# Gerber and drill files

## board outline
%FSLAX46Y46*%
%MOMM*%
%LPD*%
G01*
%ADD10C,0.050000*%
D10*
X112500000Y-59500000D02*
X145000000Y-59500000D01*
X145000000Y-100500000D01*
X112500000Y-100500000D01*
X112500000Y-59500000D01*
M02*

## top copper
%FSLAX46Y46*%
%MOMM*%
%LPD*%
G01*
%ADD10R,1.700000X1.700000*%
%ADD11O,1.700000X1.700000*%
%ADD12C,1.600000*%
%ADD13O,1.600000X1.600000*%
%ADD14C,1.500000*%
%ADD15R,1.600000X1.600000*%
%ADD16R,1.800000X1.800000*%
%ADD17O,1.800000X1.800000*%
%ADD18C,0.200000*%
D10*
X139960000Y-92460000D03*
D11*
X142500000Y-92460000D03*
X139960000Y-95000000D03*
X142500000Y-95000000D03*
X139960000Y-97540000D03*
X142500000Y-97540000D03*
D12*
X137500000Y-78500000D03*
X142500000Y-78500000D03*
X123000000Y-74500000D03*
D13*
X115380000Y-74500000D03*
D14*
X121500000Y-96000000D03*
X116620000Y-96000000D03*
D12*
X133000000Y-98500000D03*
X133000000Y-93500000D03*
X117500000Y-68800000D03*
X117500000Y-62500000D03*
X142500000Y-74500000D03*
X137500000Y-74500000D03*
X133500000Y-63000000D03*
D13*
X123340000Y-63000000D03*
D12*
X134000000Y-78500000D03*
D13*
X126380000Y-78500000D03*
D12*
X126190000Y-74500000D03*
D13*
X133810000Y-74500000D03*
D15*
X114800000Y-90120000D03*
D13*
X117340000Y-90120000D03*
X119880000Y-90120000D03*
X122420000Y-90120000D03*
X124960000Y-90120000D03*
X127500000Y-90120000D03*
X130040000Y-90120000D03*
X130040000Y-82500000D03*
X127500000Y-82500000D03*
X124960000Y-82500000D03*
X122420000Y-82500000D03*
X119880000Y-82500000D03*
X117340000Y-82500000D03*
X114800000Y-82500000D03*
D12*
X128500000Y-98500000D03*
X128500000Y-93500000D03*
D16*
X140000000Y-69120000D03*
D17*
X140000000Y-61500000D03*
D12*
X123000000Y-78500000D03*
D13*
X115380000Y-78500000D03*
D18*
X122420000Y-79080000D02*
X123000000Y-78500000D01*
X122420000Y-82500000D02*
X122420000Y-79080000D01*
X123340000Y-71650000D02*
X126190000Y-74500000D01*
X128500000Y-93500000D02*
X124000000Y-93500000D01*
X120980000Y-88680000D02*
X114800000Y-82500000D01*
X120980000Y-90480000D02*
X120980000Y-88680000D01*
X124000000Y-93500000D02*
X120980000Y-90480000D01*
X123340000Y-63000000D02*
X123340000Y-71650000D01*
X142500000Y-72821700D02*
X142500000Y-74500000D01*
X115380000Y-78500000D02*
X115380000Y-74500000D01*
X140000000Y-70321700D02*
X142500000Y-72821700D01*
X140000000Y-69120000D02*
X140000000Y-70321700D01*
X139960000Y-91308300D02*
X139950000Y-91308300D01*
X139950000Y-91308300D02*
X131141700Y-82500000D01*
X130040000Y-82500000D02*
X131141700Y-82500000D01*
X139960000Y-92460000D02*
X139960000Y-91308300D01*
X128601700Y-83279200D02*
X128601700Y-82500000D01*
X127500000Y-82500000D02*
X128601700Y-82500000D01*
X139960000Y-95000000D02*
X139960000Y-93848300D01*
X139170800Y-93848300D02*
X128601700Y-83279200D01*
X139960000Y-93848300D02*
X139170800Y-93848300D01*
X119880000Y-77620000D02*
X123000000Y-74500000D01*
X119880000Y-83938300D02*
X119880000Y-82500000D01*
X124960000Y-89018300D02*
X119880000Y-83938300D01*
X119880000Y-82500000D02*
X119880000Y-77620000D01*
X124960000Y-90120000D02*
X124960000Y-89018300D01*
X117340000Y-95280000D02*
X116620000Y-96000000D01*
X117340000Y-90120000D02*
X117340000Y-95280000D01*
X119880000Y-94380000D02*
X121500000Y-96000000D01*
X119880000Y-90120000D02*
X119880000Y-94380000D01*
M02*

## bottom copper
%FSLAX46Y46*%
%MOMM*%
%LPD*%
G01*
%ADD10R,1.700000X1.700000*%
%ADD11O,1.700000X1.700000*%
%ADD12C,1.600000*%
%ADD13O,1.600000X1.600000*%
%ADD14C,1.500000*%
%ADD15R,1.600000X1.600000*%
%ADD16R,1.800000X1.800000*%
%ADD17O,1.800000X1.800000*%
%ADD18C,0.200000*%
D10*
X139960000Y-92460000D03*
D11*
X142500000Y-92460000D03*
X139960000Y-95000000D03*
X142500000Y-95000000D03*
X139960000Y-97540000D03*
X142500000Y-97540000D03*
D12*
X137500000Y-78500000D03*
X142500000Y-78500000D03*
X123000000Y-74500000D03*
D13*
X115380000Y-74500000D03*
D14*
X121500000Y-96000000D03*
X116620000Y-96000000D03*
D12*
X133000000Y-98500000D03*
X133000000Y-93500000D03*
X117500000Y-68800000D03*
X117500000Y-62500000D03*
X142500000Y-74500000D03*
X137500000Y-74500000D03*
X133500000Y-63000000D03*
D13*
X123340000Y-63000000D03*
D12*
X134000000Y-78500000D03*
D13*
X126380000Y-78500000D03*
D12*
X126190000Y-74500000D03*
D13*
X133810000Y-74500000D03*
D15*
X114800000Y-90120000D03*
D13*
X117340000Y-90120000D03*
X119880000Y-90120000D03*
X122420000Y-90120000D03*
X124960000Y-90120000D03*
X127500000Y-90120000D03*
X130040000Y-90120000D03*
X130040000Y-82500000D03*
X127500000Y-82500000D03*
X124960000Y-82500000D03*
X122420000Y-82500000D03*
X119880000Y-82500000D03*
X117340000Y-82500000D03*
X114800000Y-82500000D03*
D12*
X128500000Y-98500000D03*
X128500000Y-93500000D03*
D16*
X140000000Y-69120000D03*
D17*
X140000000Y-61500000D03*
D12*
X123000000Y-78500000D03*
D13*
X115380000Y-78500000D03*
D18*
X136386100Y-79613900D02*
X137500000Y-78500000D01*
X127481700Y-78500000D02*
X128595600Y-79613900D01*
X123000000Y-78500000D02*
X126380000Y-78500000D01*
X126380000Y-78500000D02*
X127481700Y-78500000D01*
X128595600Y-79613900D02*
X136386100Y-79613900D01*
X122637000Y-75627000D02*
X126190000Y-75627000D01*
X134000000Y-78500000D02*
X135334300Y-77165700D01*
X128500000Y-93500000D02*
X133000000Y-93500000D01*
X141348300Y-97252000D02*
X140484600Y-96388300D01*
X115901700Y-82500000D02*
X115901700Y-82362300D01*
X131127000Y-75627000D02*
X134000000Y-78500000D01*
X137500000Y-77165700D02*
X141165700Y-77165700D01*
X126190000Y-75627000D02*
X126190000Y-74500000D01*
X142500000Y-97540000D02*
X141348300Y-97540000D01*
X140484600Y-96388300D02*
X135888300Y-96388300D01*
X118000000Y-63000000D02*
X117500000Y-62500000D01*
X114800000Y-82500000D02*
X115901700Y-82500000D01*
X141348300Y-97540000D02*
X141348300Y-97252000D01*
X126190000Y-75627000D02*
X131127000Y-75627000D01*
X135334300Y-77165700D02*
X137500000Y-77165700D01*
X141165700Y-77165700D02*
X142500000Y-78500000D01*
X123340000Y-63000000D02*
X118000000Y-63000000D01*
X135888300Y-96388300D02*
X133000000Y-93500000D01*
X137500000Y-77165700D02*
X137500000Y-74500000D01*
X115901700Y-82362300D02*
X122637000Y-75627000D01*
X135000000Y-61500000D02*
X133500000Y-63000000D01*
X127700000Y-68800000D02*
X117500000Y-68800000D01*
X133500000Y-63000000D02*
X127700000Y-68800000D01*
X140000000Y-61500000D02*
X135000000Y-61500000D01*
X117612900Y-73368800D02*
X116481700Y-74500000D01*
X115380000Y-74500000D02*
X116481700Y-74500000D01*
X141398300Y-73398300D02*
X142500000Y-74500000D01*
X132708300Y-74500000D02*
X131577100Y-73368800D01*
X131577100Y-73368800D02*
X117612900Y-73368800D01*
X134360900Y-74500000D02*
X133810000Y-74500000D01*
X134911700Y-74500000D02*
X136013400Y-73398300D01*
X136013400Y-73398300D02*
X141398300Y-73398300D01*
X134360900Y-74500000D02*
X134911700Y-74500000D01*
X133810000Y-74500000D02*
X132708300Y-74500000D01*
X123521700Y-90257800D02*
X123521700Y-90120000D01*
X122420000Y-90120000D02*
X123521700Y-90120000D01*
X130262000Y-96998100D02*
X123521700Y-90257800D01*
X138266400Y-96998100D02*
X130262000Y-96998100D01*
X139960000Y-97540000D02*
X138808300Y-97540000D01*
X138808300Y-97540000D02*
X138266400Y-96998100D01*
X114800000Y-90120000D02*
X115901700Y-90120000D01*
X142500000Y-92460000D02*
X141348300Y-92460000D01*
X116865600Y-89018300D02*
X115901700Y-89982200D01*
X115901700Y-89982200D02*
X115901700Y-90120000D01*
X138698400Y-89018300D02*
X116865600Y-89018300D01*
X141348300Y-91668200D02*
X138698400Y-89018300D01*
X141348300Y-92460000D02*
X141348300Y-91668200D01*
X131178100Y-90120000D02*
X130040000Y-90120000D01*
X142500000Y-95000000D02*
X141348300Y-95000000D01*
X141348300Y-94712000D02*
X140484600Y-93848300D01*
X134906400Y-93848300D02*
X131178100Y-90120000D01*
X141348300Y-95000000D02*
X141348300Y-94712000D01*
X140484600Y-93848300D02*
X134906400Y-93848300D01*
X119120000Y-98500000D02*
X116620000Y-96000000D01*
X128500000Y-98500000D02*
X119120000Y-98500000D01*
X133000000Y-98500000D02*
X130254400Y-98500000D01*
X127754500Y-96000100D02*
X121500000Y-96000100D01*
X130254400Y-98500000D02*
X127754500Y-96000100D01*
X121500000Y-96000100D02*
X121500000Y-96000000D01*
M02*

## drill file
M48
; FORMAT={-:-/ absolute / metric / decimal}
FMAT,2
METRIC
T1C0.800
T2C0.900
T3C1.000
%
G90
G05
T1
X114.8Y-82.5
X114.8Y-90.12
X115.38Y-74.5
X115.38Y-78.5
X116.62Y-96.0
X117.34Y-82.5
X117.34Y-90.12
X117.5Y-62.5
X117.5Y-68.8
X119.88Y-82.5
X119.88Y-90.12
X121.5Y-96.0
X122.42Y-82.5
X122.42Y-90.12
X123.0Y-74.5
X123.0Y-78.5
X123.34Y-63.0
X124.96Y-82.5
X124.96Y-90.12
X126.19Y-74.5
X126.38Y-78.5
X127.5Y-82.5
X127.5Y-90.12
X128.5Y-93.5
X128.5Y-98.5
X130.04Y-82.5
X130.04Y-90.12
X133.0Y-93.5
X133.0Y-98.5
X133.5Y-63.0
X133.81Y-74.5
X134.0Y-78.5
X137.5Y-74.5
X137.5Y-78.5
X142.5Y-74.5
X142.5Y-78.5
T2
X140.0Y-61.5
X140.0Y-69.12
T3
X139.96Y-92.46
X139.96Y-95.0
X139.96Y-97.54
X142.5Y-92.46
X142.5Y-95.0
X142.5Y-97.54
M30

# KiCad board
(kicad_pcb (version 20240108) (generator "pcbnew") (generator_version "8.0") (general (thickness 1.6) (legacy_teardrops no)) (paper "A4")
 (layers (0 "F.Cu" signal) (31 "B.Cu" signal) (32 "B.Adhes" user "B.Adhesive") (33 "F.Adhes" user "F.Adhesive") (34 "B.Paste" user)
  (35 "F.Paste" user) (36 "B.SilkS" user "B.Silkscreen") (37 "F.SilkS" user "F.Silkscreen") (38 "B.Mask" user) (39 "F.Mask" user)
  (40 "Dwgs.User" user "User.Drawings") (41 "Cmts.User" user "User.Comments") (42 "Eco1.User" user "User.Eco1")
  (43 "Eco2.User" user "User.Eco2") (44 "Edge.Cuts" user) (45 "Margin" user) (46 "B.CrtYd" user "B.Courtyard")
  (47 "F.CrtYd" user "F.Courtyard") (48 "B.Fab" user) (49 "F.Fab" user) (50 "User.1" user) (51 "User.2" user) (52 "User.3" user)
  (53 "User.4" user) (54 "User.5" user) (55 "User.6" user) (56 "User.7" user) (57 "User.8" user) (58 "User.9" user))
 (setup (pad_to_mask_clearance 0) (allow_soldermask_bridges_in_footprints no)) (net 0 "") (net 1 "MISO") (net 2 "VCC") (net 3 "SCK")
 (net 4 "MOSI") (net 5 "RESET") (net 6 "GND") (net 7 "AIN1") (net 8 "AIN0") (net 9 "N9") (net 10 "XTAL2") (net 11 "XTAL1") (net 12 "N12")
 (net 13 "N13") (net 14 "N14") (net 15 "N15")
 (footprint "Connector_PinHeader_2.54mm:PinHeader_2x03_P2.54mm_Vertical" (layer "F.Cu") (at 139.96 92.46)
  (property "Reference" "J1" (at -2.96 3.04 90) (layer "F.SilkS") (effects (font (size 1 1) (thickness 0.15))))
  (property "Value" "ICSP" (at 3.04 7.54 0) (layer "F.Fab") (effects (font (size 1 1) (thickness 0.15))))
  (pad "1" thru_hole rect (at 0 0) (size 1.7 1.7) (drill 1) (layers "*.Cu" "*.Mask") (remove_unused_layers no) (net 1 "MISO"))
  (pad "2" thru_hole oval (at 2.54 0) (size 1.7 1.7) (drill 1) (layers "*.Cu" "*.Mask") (remove_unused_layers no) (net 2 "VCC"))
  (pad "3" thru_hole oval (at 0 2.54) (size 1.7 1.7) (drill 1) (layers "*.Cu" "*.Mask") (remove_unused_layers no) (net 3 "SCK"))
  (pad "4" thru_hole oval (at 2.54 2.54) (size 1.7 1.7) (drill 1) (layers "*.Cu" "*.Mask") (remove_unused_layers no) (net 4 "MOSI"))
  (pad "5" thru_hole oval (at 0 5.08) (size 1.7 1.7) (drill 1) (layers "*.Cu" "*.Mask") (remove_unused_layers no) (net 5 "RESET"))
  (pad "6" thru_hole oval (at 2.54 5.08) (size 1.7 1.7) (drill 1) (layers "*.Cu" "*.Mask") (remove_unused_layers no) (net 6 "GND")))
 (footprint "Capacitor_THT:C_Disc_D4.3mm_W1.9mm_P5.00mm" (layer "F.Cu") (at 137.5 78.5)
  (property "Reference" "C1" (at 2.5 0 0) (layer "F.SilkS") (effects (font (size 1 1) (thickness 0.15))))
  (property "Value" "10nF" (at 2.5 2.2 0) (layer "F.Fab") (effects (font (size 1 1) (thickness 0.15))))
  (pad "1" thru_hole circle (at 0 0) (size 1.6 1.6) (drill 0.8) (layers "*.Cu" "*.Mask") (remove_unused_layers no) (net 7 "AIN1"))
  (pad "2" thru_hole circle (at 5 0) (size 1.6 1.6) (drill 0.8) (layers "*.Cu" "*.Mask") (remove_unused_layers no) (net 6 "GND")))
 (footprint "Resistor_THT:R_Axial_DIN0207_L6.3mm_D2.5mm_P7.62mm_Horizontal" (layer "F.Cu") (at 123 74.5 180)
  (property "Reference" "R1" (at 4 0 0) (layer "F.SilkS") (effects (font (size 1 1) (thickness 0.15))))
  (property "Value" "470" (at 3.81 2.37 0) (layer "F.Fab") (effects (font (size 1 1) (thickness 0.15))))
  (pad "1" thru_hole circle (at 0 0 180) (size 1.6 1.6) (drill 0.8) (layers "*.Cu" "*.Mask") (remove_unused_layers no) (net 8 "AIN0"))
  (pad "2" thru_hole oval (at 7.62 0 180) (size 1.6 1.6) (drill 0.8) (layers "*.Cu" "*.Mask") (remove_unused_layers no) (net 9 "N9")))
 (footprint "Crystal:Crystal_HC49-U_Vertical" (layer "F.Cu") (at 121.5 96 180)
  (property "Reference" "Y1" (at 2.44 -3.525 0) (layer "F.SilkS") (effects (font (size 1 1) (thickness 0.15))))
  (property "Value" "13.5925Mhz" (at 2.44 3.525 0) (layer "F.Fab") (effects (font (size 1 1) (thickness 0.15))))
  (pad "1" thru_hole circle (at 0 0 180) (size 1.5 1.5) (drill 0.8) (layers "*.Cu" "*.Mask") (remove_unused_layers no) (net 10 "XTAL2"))
  (pad "2" thru_hole circle (at 4.88 0 180) (size 1.5 1.5) (drill 0.8) (layers "*.Cu" "*.Mask") (remove_unused_layers no) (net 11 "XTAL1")))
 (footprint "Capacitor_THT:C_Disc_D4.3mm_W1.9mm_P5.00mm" (layer "F.Cu") (at 133 98.5 90)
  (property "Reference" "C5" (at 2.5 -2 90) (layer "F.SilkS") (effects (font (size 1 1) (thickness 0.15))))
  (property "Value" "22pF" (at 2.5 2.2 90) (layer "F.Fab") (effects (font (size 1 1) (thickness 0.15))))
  (pad "1" thru_hole circle (at 0 0 90) (size 1.6 1.6) (drill 0.8) (layers "*.Cu" "*.Mask") (remove_unused_layers no) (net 10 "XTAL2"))
  (pad "2" thru_hole circle (at 5 0 90) (size 1.6 1.6) (drill 0.8) (layers "*.Cu" "*.Mask") (remove_unused_layers no) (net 6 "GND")))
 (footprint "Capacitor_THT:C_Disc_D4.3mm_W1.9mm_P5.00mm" (layer "F.Cu") (at 117.5 68.2 90)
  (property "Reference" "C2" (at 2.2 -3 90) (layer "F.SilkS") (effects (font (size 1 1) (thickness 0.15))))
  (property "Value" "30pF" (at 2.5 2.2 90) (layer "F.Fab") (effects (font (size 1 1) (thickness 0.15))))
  (pad "1" thru_hole circle (at -0.6 0 90) (size 1.6 1.6) (drill 0.8) (layers "*.Cu" "*.Mask") (remove_unused_layers no) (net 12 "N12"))
  (pad "2" thru_hole circle (at 5.7 0 90) (size 1.6 1.6) (drill 0.8) (layers "*.Cu" "*.Mask") (remove_unused_layers no) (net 6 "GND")))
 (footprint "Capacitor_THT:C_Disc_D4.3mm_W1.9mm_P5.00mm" (layer "F.Cu") (at 142.5 74.5 180)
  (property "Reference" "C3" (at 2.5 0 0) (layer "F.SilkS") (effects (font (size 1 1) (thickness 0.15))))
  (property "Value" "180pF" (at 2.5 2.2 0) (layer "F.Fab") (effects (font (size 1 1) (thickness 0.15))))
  (pad "1" thru_hole circle (at 0 0 180) (size 1.6 1.6) (drill 0.8) (layers "*.Cu" "*.Mask") (remove_unused_layers no) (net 9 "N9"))
  (pad "2" thru_hole circle (at 5 0 180) (size 1.6 1.6) (drill 0.8) (layers "*.Cu" "*.Mask") (remove_unused_layers no) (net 6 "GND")))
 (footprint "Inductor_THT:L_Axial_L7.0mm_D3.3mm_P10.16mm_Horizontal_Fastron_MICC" (layer "F.Cu") (at 133.5 63 180)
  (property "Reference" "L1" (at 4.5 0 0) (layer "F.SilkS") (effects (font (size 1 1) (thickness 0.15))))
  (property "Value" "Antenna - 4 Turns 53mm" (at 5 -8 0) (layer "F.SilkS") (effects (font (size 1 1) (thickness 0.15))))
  (pad "1" thru_hole circle (at 0 0 180) (size 1.6 1.6) (drill 0.8) (layers "*.Cu" "*.Mask") (remove_unused_layers no) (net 12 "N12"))
  (pad "2" thru_hole oval (at 10.16 0 180) (size 1.6 1.6) (drill 0.8) (layers "*.Cu" "*.Mask") (remove_unused_layers no) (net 6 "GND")))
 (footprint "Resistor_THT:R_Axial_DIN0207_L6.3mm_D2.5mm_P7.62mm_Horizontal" (layer "F.Cu") (at 134 78.5 180)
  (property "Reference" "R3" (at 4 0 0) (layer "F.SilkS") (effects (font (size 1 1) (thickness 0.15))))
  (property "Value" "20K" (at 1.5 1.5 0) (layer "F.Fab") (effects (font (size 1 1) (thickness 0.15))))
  (pad "1" thru_hole circle (at 0 0 180) (size 1.6 1.6) (drill 0.8) (layers "*.Cu" "*.Mask") (remove_unused_layers no) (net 6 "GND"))
  (pad "2" thru_hole oval (at 7.62 0 180) (size 1.6 1.6) (drill 0.8) (layers "*.Cu" "*.Mask") (remove_unused_layers no) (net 7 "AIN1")))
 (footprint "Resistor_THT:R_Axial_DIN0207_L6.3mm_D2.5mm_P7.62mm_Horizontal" (layer "F.Cu") (at 126.19 74.5)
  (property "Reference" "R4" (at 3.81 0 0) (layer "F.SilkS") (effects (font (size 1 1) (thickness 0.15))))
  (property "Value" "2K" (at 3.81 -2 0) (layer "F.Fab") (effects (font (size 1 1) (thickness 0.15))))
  (pad "1" thru_hole circle (at 0 0) (size 1.6 1.6) (drill 0.8) (layers "*.Cu" "*.Mask") (remove_unused_layers no) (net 6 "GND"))
  (pad "2" thru_hole oval (at 7.62 0) (size 1.6 1.6) (drill 0.8) (layers "*.Cu" "*.Mask") (remove_unused_layers no) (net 9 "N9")))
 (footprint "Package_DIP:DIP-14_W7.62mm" (layer "F.Cu") (at 114.8 90.12 90)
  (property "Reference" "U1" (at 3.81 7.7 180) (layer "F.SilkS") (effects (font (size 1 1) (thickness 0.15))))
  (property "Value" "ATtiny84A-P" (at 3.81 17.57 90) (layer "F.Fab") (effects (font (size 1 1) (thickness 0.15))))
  (pad "1" thru_hole rect (at 0 0 90) (size 1.6 1.6) (drill 0.8) (layers "*.Cu" "*.Mask") (remove_unused_layers no) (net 2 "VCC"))
  (pad "2" thru_hole oval (at 0 2.54 90) (size 1.6 1.6) (drill 0.8) (layers "*.Cu" "*.Mask") (remove_unused_layers no) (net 11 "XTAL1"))
  (pad "3" thru_hole oval (at 0 5.08 90) (size 1.6 1.6) (drill 0.8) (layers "*.Cu" "*.Mask") (remove_unused_layers no) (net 10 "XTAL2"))
  (pad "4" thru_hole oval (at 0 7.62 90) (size 1.6 1.6) (drill 0.8) (layers "*.Cu" "*.Mask") (remove_unused_layers no) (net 5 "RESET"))
  (pad "5" thru_hole oval (at 0 10.16 90) (size 1.6 1.6) (drill 0.8) (layers "*.Cu" "*.Mask") (remove_unused_layers no) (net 8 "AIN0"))
  (pad "6" thru_hole oval (at 0 12.7 90) (size 1.6 1.6) (drill 0.8) (layers "*.Cu" "*.Mask") (remove_unused_layers no) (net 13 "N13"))
  (pad "7" thru_hole oval (at 0 15.24 90) (size 1.6 1.6) (drill 0.8) (layers "*.Cu" "*.Mask") (remove_unused_layers no) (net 4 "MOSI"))
  (pad "8" thru_hole oval (at 7.62 15.24 90) (size 1.6 1.6) (drill 0.8) (layers "*.Cu" "*.Mask") (remove_unused_layers no) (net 1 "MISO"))
  (pad "9" thru_hole oval (at 7.62 12.7 90) (size 1.6 1.6) (drill 0.8) (layers "*.Cu" "*.Mask") (remove_unused_layers no) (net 3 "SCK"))
  (pad "10" thru_hole oval (at 7.62 10.16 90) (size 1.6 1.6) (drill 0.8) (layers "*.Cu" "*.Mask") (remove_unused_layers no) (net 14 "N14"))
  (pad "11" thru_hole oval (at 7.62 7.62 90) (size 1.6 1.6) (drill 0.8) (layers "*.Cu" "*.Mask") (remove_unused_layers no) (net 7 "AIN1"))
  (pad "12" thru_hole oval (at 7.62 5.08 90) (size 1.6 1.6) (drill 0.8) (layers "*.Cu" "*.Mask") (remove_unused_layers no) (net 8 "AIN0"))
  (pad "13" thru_hole oval (at 7.62 2.54 90) (size 1.6 1.6) (drill 0.8) (layers "*.Cu" "*.Mask") (remove_unused_layers no) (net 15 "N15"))
  (pad "14" thru_hole oval (at 7.62 0 90) (size 1.6 1.6) (drill 0.8) (layers "*.Cu" "*.Mask") (remove_unused_layers no) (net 6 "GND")))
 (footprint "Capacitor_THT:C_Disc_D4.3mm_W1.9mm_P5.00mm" (layer "F.Cu") (at 128.5 98.5 90)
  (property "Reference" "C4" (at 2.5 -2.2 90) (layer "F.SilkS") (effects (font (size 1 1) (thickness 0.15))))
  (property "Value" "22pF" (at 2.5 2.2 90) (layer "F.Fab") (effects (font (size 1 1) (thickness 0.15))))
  (pad "1" thru_hole circle (at 0 0 90) (size 1.6 1.6) (drill 0.8) (layers "*.Cu" "*.Mask") (remove_unused_layers no) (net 11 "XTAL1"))
  (pad "2" thru_hole circle (at 5 0 90) (size 1.6 1.6) (drill 0.8) (layers "*.Cu" "*.Mask") (remove_unused_layers no) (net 6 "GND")))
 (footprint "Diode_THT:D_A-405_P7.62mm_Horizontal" (layer "F.Cu") (at 140 69.12 90)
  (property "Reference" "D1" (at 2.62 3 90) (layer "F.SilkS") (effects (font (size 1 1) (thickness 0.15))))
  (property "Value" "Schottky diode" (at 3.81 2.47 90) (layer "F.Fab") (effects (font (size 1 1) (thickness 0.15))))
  (pad "1" thru_hole rect (at 0 0 90) (size 1.8 1.8) (drill 0.9) (layers "*.Cu" "*.Mask") (remove_unused_layers no) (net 9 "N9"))
  (pad "2" thru_hole oval (at 7.62 0 90) (size 1.8 1.8) (drill 0.9) (layers "*.Cu" "*.Mask") (remove_unused_layers no) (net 12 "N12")))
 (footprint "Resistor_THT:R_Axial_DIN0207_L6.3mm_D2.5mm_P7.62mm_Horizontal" (layer "F.Cu") (at 123 78.5 180)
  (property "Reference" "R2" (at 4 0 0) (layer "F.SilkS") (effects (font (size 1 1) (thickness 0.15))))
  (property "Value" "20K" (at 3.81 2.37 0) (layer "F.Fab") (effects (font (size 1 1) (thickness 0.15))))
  (pad "1" thru_hole circle (at 0 0 180) (size 1.6 1.6) (drill 0.8) (layers "*.Cu" "*.Mask") (remove_unused_layers no) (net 7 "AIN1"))
  (pad "2" thru_hole oval (at 7.62 0 180) (size 1.6 1.6) (drill 0.8) (layers "*.Cu" "*.Mask") (remove_unused_layers no) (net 9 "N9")))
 (gr_rect (start 112.5 59.5) (end 145 100.5) (stroke (width 0.05) (type default)) (fill none) (layer "Edge.Cuts"))
 (segment (start 122.42 79.08) (end 123 78.5) (width 0.2) (layer "F.Cu") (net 7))
 (segment (start 122.42 82.5) (end 122.42 79.08) (width 0.2) (layer "F.Cu") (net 7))
 (segment (start 136.3861 79.6139) (end 137.5 78.5) (width 0.2) (layer "B.Cu") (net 7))
 (segment (start 127.4817 78.5) (end 128.5956 79.6139) (width 0.2) (layer "B.Cu") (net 7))
 (segment (start 123 78.5) (end 126.38 78.5) (width 0.2) (layer "B.Cu") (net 7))
 (segment (start 126.38 78.5) (end 127.4817 78.5) (width 0.2) (layer "B.Cu") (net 7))
 (segment (start 128.5956 79.6139) (end 136.3861 79.6139) (width 0.2) (layer "B.Cu") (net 7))
 (segment (start 123.34 71.65) (end 126.19 74.5) (width 0.2) (layer "F.Cu") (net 6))
 (segment (start 128.5 93.5) (end 124 93.5) (width 0.2) (layer "F.Cu") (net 6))
 (segment (start 120.98 88.68) (end 114.8 82.5) (width 0.2) (layer "F.Cu") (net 6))
 (segment (start 120.98 90.48) (end 120.98 88.68) (width 0.2) (layer "F.Cu") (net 6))
 (segment (start 124 93.5) (end 120.98 90.48) (width 0.2) (layer "F.Cu") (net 6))
 (segment (start 123.34 63) (end 123.34 71.65) (width 0.2) (layer "F.Cu") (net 6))
 (segment (start 122.637 75.627) (end 126.19 75.627) (width 0.2) (layer "B.Cu") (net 6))
 (segment (start 134 78.5) (end 135.3343 77.1657) (width 0.2) (layer "B.Cu") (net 6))
 (segment (start 128.5 93.5) (end 133 93.5) (width 0.2) (layer "B.Cu") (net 6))
 (segment (start 141.3483 97.252) (end 140.4846 96.3883) (width 0.2) (layer "B.Cu") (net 6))
 (segment (start 115.9017 82.5) (end 115.9017 82.3623) (width 0.2) (layer "B.Cu") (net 6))
 (segment (start 131.127 75.627) (end 134 78.5) (width 0.2) (layer "B.Cu") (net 6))
 (segment (start 137.5 77.1657) (end 141.1657 77.1657) (width 0.2) (layer "B.Cu") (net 6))
 (segment (start 126.19 75.627) (end 126.19 74.5) (width 0.2) (layer "B.Cu") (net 6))
 (segment (start 142.5 97.54) (end 141.3483 97.54) (width 0.2) (layer "B.Cu") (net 6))
 (segment (start 140.4846 96.3883) (end 135.8883 96.3883) (width 0.2) (layer "B.Cu") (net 6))
 (segment (start 118 63) (end 117.5 62.5) (width 0.2) (layer "B.Cu") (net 6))
 (segment (start 114.8 82.5) (end 115.9017 82.5) (width 0.2) (layer "B.Cu") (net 6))
 (segment (start 141.3483 97.54) (end 141.3483 97.252) (width 0.2) (layer "B.Cu") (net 6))
 (segment (start 126.19 75.627) (end 131.127 75.627) (width 0.2) (layer "B.Cu") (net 6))
 (segment (start 135.3343 77.1657) (end 137.5 77.1657) (width 0.2) (layer "B.Cu") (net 6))
 (segment (start 141.1657 77.1657) (end 142.5 78.5) (width 0.2) (layer "B.Cu") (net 6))
 (segment (start 123.34 63) (end 118 63) (width 0.2) (layer "B.Cu") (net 6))
 (segment (start 135.8883 96.3883) (end 133 93.5) (width 0.2) (layer "B.Cu") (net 6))
 (segment (start 137.5 77.1657) (end 137.5 74.5) (width 0.2) (layer "B.Cu") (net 6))
 (segment (start 115.9017 82.3623) (end 122.637 75.627) (width 0.2) (layer "B.Cu") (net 6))
 (segment (start 135 61.5) (end 133.5 63) (width 0.2) (layer "B.Cu") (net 12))
 (segment (start 127.7 68.8) (end 117.5 68.8) (width 0.2) (layer "B.Cu") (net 12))
 (segment (start 133.5 63) (end 127.7 68.8) (width 0.2) (layer "B.Cu") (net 12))
 (segment (start 140 61.5) (end 135 61.5) (width 0.2) (layer "B.Cu") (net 12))
 (segment (start 142.5 72.8217) (end 142.5 74.5) (width 0.2) (layer "F.Cu") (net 9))
 (segment (start 115.38 78.5) (end 115.38 74.5) (width 0.2) (layer "F.Cu") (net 9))
 (segment (start 140 70.3217) (end 142.5 72.8217) (width 0.2) (layer "F.Cu") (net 9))
 (segment (start 140 69.12) (end 140 70.3217) (width 0.2) (layer "F.Cu") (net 9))
 (segment (start 117.6129 73.3688) (end 116.4817 74.5) (width 0.2) (layer "B.Cu") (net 9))
 (segment (start 115.38 74.5) (end 116.4817 74.5) (width 0.2) (layer "B.Cu") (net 9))
 (segment (start 141.3983 73.3983) (end 142.5 74.5) (width 0.2) (layer "B.Cu") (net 9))
 (segment (start 132.7083 74.5) (end 131.5771 73.3688) (width 0.2) (layer "B.Cu") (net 9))
 (segment (start 131.5771 73.3688) (end 117.6129 73.3688) (width 0.2) (layer "B.Cu") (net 9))
 (segment (start 134.3609 74.5) (end 133.81 74.5) (width 0.2) (layer "B.Cu") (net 9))
 (segment (start 134.9117 74.5) (end 136.0134 73.3983) (width 0.2) (layer "B.Cu") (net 9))
 (segment (start 136.0134 73.3983) (end 141.3983 73.3983) (width 0.2) (layer "B.Cu") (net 9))
 (segment (start 134.3609 74.5) (end 134.9117 74.5) (width 0.2) (layer "B.Cu") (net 9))
 (segment (start 133.81 74.5) (end 132.7083 74.5) (width 0.2) (layer "B.Cu") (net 9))
 (segment (start 139.96 91.3083) (end 139.95 91.3083) (width 0.2) (layer "F.Cu") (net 1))
 (segment (start 139.95 91.3083) (end 131.1417 82.5) (width 0.2) (layer "F.Cu") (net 1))
 (segment (start 130.04 82.5) (end 131.1417 82.5) (width 0.2) (layer "F.Cu") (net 1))
 (segment (start 139.96 92.46) (end 139.96 91.3083) (width 0.2) (layer "F.Cu") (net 1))
 (segment (start 123.5217 90.2578) (end 123.5217 90.12) (width 0.2) (layer "B.Cu") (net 5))
 (segment (start 122.42 90.12) (end 123.5217 90.12) (width 0.2) (layer "B.Cu") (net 5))
 (segment (start 130.262 96.9981) (end 123.5217 90.2578) (width 0.2) (layer "B.Cu") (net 5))
 (segment (start 138.2664 96.9981) (end 130.262 96.9981) (width 0.2) (layer "B.Cu") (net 5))
 (segment (start 139.96 97.54) (end 138.8083 97.54) (width 0.2) (layer "B.Cu") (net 5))
 (segment (start 138.8083 97.54) (end 138.2664 96.9981) (width 0.2) (layer "B.Cu") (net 5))
 (segment (start 128.6017 83.2792) (end 128.6017 82.5) (width 0.2) (layer "F.Cu") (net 3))
 (segment (start 127.5 82.5) (end 128.6017 82.5) (width 0.2) (layer "F.Cu") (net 3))
 (segment (start 139.96 95) (end 139.96 93.8483) (width 0.2) (layer "F.Cu") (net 3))
 (segment (start 139.1708 93.8483) (end 128.6017 83.2792) (width 0.2) (layer "F.Cu") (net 3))
 (segment (start 139.96 93.8483) (end 139.1708 93.8483) (width 0.2) (layer "F.Cu") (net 3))
 (segment (start 114.8 90.12) (end 115.9017 90.12) (width 0.2) (layer "B.Cu") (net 2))
 (segment (start 142.5 92.46) (end 141.3483 92.46) (width 0.2) (layer "B.Cu") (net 2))
 (segment (start 116.8656 89.0183) (end 115.9017 89.9822) (width 0.2) (layer "B.Cu") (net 2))
 (segment (start 115.9017 89.9822) (end 115.9017 90.12) (width 0.2) (layer "B.Cu") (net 2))
 (segment (start 138.6984 89.0183) (end 116.8656 89.0183) (width 0.2) (layer "B.Cu") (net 2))
 (segment (start 141.3483 91.6682) (end 138.6984 89.0183) (width 0.2) (layer "B.Cu") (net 2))
 (segment (start 141.3483 92.46) (end 141.3483 91.6682) (width 0.2) (layer "B.Cu") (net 2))
 (segment (start 131.1781 90.12) (end 130.04 90.12) (width 0.2) (layer "B.Cu") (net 4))
 (segment (start 142.5 95) (end 141.3483 95) (width 0.2) (layer "B.Cu") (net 4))
 (segment (start 141.3483 94.712) (end 140.4846 93.8483) (width 0.2) (layer "B.Cu") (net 4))
 (segment (start 134.9064 93.8483) (end 131.1781 90.12) (width 0.2) (layer "B.Cu") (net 4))
 (segment (start 141.3483 95) (end 141.3483 94.712) (width 0.2) (layer "B.Cu") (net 4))
 (segment (start 140.4846 93.8483) (end 134.9064 93.8483) (width 0.2) (layer "B.Cu") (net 4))
 (segment (start 119.88 77.62) (end 123 74.5) (width 0.2) (layer "F.Cu") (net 8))
 (segment (start 119.88 83.9383) (end 119.88 82.5) (width 0.2) (layer "F.Cu") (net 8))
 (segment (start 124.96 89.0183) (end 119.88 83.9383) (width 0.2) (layer "F.Cu") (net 8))
 (segment (start 119.88 82.5) (end 119.88 77.62) (width 0.2) (layer "F.Cu") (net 8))
 (segment (start 124.96 90.12) (end 124.96 89.0183) (width 0.2) (layer "F.Cu") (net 8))
 (segment (start 117.34 95.28) (end 116.62 96) (width 0.2) (layer "F.Cu") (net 11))
 (segment (start 117.34 90.12) (end 117.34 95.28) (width 0.2) (layer "F.Cu") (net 11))
 (segment (start 119.12 98.5) (end 116.62 96) (width 0.2) (layer "B.Cu") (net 11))
 (segment (start 128.5 98.5) (end 119.12 98.5) (width 0.2) (layer "B.Cu") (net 11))
 (segment (start 119.88 94.38) (end 121.5 96) (width 0.2) (layer "F.Cu") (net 10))
 (segment (start 119.88 90.12) (end 119.88 94.38) (width 0.2) (layer "F.Cu") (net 10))
 (segment (start 133 98.5) (end 130.2544 98.5) (width 0.2) (layer "B.Cu") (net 10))
 (segment (start 127.7545 96.0001) (end 121.5 96.0001) (width 0.2) (layer "B.Cu") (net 10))
 (segment (start 130.2544 98.5) (end 127.7545 96.0001) (width 0.2) (layer "B.Cu") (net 10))
 (segment (start 121.5 96.0001) (end 121.5 96) (width 0.2) (layer "B.Cu") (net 10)))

